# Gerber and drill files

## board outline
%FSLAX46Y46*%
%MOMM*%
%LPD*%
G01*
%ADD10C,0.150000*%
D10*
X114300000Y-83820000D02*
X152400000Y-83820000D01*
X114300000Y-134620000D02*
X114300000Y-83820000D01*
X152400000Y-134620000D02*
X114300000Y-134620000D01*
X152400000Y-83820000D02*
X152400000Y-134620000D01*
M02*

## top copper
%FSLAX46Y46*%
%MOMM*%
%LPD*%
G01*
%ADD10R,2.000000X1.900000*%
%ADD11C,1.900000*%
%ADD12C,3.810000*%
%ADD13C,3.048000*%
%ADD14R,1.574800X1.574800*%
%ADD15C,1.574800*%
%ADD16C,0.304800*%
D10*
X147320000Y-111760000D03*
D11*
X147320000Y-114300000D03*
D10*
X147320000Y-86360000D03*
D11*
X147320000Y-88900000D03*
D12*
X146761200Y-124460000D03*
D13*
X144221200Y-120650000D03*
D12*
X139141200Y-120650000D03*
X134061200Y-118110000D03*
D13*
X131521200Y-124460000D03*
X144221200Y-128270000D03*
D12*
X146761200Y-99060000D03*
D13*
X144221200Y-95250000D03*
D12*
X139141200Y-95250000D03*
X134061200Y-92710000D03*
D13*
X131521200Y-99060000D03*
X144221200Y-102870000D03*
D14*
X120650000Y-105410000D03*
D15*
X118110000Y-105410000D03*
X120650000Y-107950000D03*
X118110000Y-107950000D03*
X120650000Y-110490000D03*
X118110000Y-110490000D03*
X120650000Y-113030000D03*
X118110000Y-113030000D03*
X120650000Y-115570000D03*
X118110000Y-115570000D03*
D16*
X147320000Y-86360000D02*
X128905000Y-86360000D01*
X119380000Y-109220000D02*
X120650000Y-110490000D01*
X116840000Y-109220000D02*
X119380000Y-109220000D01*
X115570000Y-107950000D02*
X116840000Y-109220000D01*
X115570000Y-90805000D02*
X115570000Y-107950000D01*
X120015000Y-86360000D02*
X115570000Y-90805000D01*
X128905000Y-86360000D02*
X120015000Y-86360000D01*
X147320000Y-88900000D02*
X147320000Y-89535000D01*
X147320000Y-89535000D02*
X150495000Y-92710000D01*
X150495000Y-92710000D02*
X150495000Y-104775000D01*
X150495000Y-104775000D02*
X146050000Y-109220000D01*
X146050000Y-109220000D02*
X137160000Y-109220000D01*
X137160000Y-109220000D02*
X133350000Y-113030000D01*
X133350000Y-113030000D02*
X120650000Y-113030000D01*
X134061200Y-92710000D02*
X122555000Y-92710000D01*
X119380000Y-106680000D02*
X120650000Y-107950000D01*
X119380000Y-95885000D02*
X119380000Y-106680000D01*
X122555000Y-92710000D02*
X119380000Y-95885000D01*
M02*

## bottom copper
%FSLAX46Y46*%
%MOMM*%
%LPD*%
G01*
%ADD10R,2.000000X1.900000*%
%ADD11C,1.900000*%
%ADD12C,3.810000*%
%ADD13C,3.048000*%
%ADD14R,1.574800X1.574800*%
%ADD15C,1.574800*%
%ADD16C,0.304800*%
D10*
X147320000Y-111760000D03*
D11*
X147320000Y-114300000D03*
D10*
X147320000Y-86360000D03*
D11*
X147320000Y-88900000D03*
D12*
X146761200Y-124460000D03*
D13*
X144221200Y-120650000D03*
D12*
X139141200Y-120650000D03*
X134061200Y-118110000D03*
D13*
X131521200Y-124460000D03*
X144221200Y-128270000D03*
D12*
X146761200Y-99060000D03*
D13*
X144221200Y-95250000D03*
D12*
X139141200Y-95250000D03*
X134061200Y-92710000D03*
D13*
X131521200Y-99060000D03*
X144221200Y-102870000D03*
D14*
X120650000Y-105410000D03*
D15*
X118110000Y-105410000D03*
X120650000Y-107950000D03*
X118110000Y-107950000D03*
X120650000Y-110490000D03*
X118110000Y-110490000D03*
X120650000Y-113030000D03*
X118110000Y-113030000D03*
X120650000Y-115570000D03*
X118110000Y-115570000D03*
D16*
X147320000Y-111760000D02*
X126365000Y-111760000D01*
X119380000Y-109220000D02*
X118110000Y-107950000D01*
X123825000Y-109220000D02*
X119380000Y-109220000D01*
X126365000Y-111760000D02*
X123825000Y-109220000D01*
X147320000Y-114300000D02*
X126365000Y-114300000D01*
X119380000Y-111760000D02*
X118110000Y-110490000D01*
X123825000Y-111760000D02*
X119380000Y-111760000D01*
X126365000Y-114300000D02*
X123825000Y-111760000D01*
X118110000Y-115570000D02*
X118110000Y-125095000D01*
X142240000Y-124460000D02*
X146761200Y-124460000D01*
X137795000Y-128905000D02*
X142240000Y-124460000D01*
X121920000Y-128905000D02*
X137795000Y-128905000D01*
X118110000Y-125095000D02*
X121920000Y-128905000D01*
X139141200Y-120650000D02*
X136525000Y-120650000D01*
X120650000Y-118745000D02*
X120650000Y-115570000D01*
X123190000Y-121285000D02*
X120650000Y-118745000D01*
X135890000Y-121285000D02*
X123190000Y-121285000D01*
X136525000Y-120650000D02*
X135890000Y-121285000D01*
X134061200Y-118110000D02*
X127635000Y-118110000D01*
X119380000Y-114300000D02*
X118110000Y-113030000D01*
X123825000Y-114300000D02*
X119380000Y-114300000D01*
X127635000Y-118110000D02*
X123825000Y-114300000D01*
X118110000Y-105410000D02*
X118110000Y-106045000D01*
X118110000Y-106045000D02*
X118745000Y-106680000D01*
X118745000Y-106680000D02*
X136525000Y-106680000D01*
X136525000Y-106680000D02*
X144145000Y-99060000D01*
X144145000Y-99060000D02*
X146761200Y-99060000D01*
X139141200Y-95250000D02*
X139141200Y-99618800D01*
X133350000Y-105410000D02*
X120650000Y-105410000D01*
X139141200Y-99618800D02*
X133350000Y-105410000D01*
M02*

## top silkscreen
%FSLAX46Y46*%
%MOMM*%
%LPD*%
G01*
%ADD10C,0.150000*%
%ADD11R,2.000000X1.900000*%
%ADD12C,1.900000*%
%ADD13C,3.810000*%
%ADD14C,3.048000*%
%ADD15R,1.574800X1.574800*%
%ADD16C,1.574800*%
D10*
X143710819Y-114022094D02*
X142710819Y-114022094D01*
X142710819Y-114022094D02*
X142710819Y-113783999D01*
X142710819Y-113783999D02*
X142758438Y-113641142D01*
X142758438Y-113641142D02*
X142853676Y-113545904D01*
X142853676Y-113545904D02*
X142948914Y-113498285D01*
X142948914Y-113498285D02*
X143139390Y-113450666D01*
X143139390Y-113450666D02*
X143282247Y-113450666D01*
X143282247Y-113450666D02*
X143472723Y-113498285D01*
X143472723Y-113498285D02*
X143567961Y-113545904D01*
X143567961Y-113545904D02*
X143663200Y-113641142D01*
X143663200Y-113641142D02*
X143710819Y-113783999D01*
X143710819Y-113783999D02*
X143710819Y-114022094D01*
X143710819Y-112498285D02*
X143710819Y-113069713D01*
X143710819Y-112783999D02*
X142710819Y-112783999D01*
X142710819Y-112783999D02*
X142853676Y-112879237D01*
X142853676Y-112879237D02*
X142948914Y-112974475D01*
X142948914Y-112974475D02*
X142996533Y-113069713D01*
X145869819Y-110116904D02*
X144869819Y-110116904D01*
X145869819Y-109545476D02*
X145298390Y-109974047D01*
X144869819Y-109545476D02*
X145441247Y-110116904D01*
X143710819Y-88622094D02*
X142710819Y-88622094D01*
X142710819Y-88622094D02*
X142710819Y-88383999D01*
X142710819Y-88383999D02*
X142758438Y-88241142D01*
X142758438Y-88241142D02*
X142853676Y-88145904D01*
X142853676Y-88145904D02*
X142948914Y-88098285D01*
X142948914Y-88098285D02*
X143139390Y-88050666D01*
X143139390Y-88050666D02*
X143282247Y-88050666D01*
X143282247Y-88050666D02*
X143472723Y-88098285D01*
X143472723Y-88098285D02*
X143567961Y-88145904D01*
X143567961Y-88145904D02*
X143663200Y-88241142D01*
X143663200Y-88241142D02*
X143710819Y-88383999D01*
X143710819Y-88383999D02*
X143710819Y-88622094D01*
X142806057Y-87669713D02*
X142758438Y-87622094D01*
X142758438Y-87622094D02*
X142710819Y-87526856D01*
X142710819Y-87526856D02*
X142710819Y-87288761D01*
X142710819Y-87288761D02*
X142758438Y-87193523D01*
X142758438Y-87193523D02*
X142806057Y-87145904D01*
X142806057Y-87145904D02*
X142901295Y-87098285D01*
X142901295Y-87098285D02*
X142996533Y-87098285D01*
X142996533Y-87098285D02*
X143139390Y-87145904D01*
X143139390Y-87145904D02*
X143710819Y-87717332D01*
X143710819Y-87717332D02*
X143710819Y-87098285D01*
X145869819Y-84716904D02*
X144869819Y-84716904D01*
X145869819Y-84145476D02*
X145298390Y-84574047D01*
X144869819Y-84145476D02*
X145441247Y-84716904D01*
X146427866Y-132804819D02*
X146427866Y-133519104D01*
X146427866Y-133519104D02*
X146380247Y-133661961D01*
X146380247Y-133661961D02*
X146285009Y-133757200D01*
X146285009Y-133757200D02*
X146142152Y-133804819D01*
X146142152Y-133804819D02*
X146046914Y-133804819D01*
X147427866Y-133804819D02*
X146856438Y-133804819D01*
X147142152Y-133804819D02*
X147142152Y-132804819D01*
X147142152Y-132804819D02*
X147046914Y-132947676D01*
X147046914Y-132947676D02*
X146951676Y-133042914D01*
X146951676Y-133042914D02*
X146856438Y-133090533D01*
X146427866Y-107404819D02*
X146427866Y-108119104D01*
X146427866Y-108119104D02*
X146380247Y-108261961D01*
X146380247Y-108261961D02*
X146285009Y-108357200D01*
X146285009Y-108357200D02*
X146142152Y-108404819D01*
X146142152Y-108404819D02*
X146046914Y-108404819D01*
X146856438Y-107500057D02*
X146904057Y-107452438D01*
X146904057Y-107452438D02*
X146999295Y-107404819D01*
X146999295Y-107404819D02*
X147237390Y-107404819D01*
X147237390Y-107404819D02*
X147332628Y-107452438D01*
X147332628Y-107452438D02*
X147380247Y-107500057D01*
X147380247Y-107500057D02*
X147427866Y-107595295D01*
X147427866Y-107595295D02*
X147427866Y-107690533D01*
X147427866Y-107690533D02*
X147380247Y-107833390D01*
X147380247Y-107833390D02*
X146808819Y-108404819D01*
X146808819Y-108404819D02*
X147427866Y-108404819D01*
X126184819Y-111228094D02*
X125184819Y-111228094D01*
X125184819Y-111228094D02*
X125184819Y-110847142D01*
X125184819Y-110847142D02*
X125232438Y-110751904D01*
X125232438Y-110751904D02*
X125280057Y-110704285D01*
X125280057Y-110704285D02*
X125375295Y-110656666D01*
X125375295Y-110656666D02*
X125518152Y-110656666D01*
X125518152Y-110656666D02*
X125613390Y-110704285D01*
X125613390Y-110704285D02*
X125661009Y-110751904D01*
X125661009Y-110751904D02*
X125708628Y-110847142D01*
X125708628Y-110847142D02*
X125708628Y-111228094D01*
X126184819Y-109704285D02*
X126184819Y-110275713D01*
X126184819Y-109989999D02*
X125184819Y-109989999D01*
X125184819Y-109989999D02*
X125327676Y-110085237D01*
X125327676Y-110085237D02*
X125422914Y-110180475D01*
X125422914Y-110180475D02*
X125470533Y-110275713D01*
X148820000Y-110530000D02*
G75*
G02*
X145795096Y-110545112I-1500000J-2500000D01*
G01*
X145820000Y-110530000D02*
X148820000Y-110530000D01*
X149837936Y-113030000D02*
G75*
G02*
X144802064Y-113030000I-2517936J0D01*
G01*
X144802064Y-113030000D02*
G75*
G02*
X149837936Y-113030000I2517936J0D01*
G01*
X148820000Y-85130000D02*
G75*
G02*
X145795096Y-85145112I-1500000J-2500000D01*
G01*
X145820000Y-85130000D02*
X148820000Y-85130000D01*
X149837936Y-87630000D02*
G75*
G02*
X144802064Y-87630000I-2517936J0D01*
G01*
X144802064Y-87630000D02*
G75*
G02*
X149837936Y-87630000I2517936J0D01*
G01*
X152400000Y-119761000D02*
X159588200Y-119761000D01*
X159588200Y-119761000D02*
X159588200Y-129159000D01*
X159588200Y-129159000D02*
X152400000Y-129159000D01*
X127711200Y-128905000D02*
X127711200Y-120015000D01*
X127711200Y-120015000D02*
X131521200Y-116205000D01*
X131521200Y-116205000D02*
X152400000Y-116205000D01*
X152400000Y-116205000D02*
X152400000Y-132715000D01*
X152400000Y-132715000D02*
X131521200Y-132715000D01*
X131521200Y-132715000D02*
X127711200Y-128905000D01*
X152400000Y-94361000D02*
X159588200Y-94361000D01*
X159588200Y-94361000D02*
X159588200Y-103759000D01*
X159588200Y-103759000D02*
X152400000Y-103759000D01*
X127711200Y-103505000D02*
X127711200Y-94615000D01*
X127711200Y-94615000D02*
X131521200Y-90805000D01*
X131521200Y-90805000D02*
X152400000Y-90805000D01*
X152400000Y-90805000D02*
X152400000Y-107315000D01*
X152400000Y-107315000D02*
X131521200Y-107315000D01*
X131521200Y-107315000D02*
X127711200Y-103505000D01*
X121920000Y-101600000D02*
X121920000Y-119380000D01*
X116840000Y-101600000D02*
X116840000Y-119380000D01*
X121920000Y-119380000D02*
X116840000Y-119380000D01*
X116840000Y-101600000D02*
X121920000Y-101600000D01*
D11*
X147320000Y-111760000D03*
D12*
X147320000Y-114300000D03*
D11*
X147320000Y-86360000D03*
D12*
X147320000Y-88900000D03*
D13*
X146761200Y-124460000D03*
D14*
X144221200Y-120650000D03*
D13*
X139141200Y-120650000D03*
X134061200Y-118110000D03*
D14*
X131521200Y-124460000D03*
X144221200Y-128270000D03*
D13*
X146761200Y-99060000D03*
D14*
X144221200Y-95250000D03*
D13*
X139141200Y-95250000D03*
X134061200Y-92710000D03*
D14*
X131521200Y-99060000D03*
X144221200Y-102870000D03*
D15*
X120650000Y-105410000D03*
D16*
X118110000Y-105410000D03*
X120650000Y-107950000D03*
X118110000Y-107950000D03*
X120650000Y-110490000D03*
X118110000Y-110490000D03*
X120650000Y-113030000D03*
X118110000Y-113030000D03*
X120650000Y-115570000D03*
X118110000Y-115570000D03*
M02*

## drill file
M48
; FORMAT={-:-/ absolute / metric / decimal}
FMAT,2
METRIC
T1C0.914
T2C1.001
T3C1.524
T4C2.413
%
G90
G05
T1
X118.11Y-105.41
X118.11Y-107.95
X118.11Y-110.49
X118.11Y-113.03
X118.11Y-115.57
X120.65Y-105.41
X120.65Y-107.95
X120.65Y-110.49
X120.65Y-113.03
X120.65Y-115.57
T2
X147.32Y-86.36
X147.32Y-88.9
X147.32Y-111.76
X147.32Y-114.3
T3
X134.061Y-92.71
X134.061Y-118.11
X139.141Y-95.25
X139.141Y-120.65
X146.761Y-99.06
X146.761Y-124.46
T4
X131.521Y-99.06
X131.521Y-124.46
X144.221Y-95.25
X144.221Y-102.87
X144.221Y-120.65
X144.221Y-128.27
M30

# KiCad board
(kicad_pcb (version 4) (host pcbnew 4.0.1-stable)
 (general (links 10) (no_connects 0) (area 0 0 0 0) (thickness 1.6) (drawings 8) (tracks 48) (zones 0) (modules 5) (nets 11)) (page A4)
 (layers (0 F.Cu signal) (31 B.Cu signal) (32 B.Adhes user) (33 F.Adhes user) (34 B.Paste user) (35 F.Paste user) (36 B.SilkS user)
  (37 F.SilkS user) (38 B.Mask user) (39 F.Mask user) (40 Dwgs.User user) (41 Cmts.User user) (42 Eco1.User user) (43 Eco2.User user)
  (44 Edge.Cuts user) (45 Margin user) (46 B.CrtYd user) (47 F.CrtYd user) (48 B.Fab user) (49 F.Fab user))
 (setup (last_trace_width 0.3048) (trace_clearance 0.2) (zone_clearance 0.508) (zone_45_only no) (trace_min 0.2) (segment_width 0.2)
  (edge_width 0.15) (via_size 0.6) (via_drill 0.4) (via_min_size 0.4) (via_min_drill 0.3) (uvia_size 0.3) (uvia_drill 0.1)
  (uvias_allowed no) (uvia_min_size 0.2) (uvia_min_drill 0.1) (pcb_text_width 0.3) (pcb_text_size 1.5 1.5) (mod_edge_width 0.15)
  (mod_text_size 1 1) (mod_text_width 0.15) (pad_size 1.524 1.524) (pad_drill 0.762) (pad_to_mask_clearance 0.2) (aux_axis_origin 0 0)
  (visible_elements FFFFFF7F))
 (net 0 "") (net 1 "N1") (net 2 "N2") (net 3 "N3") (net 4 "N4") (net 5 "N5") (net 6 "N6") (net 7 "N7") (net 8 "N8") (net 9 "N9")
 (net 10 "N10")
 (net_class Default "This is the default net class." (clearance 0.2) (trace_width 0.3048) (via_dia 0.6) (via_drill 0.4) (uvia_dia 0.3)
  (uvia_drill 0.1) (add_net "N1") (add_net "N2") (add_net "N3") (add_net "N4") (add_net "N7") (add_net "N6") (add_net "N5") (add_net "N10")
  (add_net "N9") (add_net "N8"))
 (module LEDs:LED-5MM (layer F.Cu) (at 147.32 111.76 270)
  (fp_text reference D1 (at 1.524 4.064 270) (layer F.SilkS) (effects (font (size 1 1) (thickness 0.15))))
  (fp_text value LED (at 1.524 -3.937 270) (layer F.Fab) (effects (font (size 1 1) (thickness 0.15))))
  (fp_arc (start 1.27 0) (end -1.23 -1.5) (angle 297.5) (layer F.SilkS) (width 0.15))
  (fp_line (start -1.23 1.5) (end -1.23 -1.5) (layer F.SilkS) (width 0.15))
  (fp_circle (center 1.27 0) (end 0.97 -2.5) (layer F.SilkS) (width 0.15))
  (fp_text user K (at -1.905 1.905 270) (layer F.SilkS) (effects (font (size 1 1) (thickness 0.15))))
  (pad 1 thru_hole rect (at 0 0) (size 2 1.9) (drill 1.00076) (layers *.Cu *.Mask F.SilkS) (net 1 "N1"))
  (pad 2 thru_hole circle (at 2.54 0 270) (size 1.9 1.9) (drill 1.00076) (layers *.Cu *.Mask F.SilkS) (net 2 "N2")))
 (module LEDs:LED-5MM (layer F.Cu) (at 147.32 86.36 270)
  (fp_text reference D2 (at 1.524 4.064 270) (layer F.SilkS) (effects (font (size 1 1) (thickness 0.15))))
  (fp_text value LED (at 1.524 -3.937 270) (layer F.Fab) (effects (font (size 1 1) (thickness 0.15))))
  (fp_arc (start 1.27 0) (end -1.23 -1.5) (angle 297.5) (layer F.SilkS) (width 0.15))
  (fp_line (start -1.23 1.5) (end -1.23 -1.5) (layer F.SilkS) (width 0.15))
  (fp_circle (center 1.27 0) (end 0.97 -2.5) (layer F.SilkS) (width 0.15))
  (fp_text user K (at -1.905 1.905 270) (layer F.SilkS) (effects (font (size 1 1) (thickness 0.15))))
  (pad 1 thru_hole rect (at 0 0) (size 2 1.9) (drill 1.00076) (layers *.Cu *.Mask F.SilkS) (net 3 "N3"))
  (pad 2 thru_hole circle (at 2.54 0 270) (size 1.9 1.9) (drill 1.00076) (layers *.Cu *.Mask F.SilkS) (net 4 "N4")))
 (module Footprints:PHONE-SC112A (layer F.Cu) (at 152.4 124.46)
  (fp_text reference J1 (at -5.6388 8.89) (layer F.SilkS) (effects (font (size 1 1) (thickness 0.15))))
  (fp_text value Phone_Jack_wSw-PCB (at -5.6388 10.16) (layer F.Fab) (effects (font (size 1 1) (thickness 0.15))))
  (fp_line (start 0 -4.699) (end 7.1882 -4.699) (layer F.SilkS) (width 0.15))
  (fp_line (start 7.1882 -4.699) (end 7.1882 4.699) (layer F.SilkS) (width 0.15))
  (fp_line (start 7.1882 4.699) (end 0 4.699) (layer F.SilkS) (width 0.15))
  (fp_line (start -24.6888 4.445) (end -24.6888 -4.445) (layer F.SilkS) (width 0.15))
  (fp_line (start -24.6888 -4.445) (end -20.8788 -8.255) (layer F.SilkS) (width 0.15))
  (fp_line (start -20.8788 -8.255) (end 0 -8.255) (layer F.SilkS) (width 0.15))
  (fp_line (start 0 -8.255) (end 0 8.255) (layer F.SilkS) (width 0.15))
  (fp_line (start 0 8.255) (end -20.8788 8.255) (layer F.SilkS) (width 0.15))
  (fp_line (start -20.8788 8.255) (end -24.6888 4.445) (layer F.SilkS) (width 0.15))
  (pad 3 thru_hole circle (at -5.6388 0) (size 3.81 3.81) (drill 1.524) (layers *.Cu *.Mask F.SilkS) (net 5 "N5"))
  (pad "" thru_hole circle (at -8.1788 -3.81) (size 3.048 3.048) (drill 2.413) (layers *.Cu *.Mask F.SilkS))
  (pad 2 thru_hole circle (at -13.2588 -3.81) (size 3.81 3.81) (drill 1.524) (layers *.Cu *.Mask F.SilkS) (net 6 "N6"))
  (pad 1 thru_hole circle (at -18.3388 -6.35) (size 3.81 3.81) (drill 1.524) (layers *.Cu *.Mask F.SilkS) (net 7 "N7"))
  (pad "" thru_hole circle (at -20.8788 0) (size 3.048 3.048) (drill 2.413) (layers *.Cu *.Mask F.SilkS))
  (pad "" thru_hole circle (at -8.1788 3.81) (size 3.048 3.048) (drill 2.413) (layers *.Cu *.Mask F.SilkS)))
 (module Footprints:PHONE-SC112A (layer F.Cu) (at 152.4 99.06)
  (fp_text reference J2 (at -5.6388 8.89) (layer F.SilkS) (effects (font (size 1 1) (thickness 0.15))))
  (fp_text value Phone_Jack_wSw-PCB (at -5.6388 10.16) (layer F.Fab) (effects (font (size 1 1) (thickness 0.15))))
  (fp_line (start 0 -4.699) (end 7.1882 -4.699) (layer F.SilkS) (width 0.15))
  (fp_line (start 7.1882 -4.699) (end 7.1882 4.699) (layer F.SilkS) (width 0.15))
  (fp_line (start 7.1882 4.699) (end 0 4.699) (layer F.SilkS) (width 0.15))
  (fp_line (start -24.6888 4.445) (end -24.6888 -4.445) (layer F.SilkS) (width 0.15))
  (fp_line (start -24.6888 -4.445) (end -20.8788 -8.255) (layer F.SilkS) (width 0.15))
  (fp_line (start -20.8788 -8.255) (end 0 -8.255) (layer F.SilkS) (width 0.15))
  (fp_line (start 0 -8.255) (end 0 8.255) (layer F.SilkS) (width 0.15))
  (fp_line (start 0 8.255) (end -20.8788 8.255) (layer F.SilkS) (width 0.15))
  (fp_line (start -20.8788 8.255) (end -24.6888 4.445) (layer F.SilkS) (width 0.15))
  (pad 3 thru_hole circle (at -5.6388 0) (size 3.81 3.81) (drill 1.524) (layers *.Cu *.Mask F.SilkS) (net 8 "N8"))
  (pad "" thru_hole circle (at -8.1788 -3.81) (size 3.048 3.048) (drill 2.413) (layers *.Cu *.Mask F.SilkS))
  (pad 2 thru_hole circle (at -13.2588 -3.81) (size 3.81 3.81) (drill 1.524) (layers *.Cu *.Mask F.SilkS) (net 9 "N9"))
  (pad 1 thru_hole circle (at -18.3388 -6.35) (size 3.81 3.81) (drill 1.524) (layers *.Cu *.Mask F.SilkS) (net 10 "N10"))
  (pad "" thru_hole circle (at -20.8788 0) (size 3.048 3.048) (drill 2.413) (layers *.Cu *.Mask F.SilkS))
  (pad "" thru_hole circle (at -8.1788 3.81) (size 3.048 3.048) (drill 2.413) (layers *.Cu *.Mask F.SilkS)))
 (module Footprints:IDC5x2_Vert (layer F.Cu) (at 119.38 114.3 90)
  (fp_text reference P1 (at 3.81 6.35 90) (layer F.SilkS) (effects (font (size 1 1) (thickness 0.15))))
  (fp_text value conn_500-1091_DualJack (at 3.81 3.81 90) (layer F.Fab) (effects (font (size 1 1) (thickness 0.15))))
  (fp_line (start 12.7 2.54) (end -5.08 2.54) (layer F.SilkS) (width 0.15))
  (fp_line (start 12.7 -2.54) (end -5.08 -2.54) (layer F.SilkS) (width 0.15))
  (fp_line (start -5.08 2.54) (end -5.08 -2.54) (layer F.SilkS) (width 0.15))
  (fp_line (start 12.7 -2.54) (end 12.7 2.54) (layer F.SilkS) (width 0.15))
  (pad 1 thru_hole rect (at 8.89 1.27 90) (size 1.5748 1.5748) (drill 0.9144) (layers *.Cu *.Mask F.SilkS) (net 9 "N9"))
  (pad 2 thru_hole circle (at 8.89 -1.27 90) (size 1.5748 1.5748) (drill 0.9144) (layers *.Cu *.Mask F.SilkS) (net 8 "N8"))
  (pad 3 thru_hole circle (at 6.35 1.27 90) (size 1.5748 1.5748) (drill 0.9144) (layers *.Cu *.Mask F.SilkS) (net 10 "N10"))
  (pad 4 thru_hole circle (at 6.35 -1.27 90) (size 1.5748 1.5748) (drill 0.9144) (layers *.Cu *.Mask F.SilkS) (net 1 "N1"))
  (pad 5 thru_hole circle (at 3.81 1.27 90) (size 1.5748 1.5748) (drill 0.9144) (layers *.Cu *.Mask F.SilkS) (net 3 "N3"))
  (pad 6 thru_hole circle (at 3.81 -1.27 90) (size 1.5748 1.5748) (drill 0.9144) (layers *.Cu *.Mask F.SilkS) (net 2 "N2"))
  (pad 7 thru_hole circle (at 1.27 1.27 90) (size 1.5748 1.5748) (drill 0.9144) (layers *.Cu *.Mask F.SilkS) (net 4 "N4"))
  (pad 8 thru_hole circle (at 1.27 -1.27 90) (size 1.5748 1.5748) (drill 0.9144) (layers *.Cu *.Mask F.SilkS) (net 7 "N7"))
  (pad 9 thru_hole circle (at -1.27 1.27 90) (size 1.5748 1.5748) (drill 0.9144) (layers *.Cu *.Mask F.SilkS) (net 6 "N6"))
  (pad 10 thru_hole circle (at -1.27 -1.27 90) (size 1.5748 1.5748) (drill 0.9144) (layers *.Cu *.Mask F.SilkS) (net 5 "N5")))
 (gr_line (start 114.3 83.82) (end 152.4 83.82) (angle 90) (layer Edge.Cuts) (width 0.15))
 (gr_line (start 114.3 134.62) (end 114.3 83.82) (angle 90) (layer Edge.Cuts) (width 0.15))
 (gr_line (start 152.4 134.62) (end 114.3 134.62) (angle 90) (layer Edge.Cuts) (width 0.15))
 (gr_line (start 152.4 83.82) (end 152.4 134.62) (angle 90) (layer Edge.Cuts) (width 0.15))
 (segment (start 147.32 111.76) (end 126.365 111.76) (width 0.3048) (layer B.Cu) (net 1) (status 400000))
 (segment (start 119.38 109.22) (end 118.11 107.95) (width 0.3048) (layer B.Cu) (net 1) (status 800000))
 (segment (start 123.825 109.22) (end 119.38 109.22) (width 0.3048) (layer B.Cu) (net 1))
 (segment (start 126.365 111.76) (end 123.825 109.22) (width 0.3048) (layer B.Cu) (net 1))
 (segment (start 147.32 114.3) (end 126.365 114.3) (width 0.3048) (layer B.Cu) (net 2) (status 400000))
 (segment (start 119.38 111.76) (end 118.11 110.49) (width 0.3048) (layer B.Cu) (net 2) (status 800000))
 (segment (start 123.825 111.76) (end 119.38 111.76) (width 0.3048) (layer B.Cu) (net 2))
 (segment (start 126.365 114.3) (end 123.825 111.76) (width 0.3048) (layer B.Cu) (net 2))
 (segment (start 147.32 86.36) (end 128.905 86.36) (width 0.3048) (layer F.Cu) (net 3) (status 400000))
 (segment (start 119.38 109.22) (end 120.65 110.49) (width 0.3048) (layer F.Cu) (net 3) (status 800000))
 (segment (start 116.84 109.22) (end 119.38 109.22) (width 0.3048) (layer F.Cu) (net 3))
 (segment (start 115.57 107.95) (end 116.84 109.22) (width 0.3048) (layer F.Cu) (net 3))
 (segment (start 115.57 90.805) (end 115.57 107.95) (width 0.3048) (layer F.Cu) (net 3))
 (segment (start 120.015 86.36) (end 115.57 90.805) (width 0.3048) (layer F.Cu) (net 3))
 (segment (start 128.905 86.36) (end 120.015 86.36) (width 0.3048) (layer F.Cu) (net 3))
 (segment (start 147.32 88.9) (end 147.32 89.535) (width 0.3048) (layer F.Cu) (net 4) (status C00000))
 (segment (start 147.32 89.535) (end 150.495 92.71) (width 0.3048) (layer F.Cu) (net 4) (status 400000))
 (segment (start 150.495 92.71) (end 150.495 104.775) (width 0.3048) (layer F.Cu) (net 4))
 (segment (start 150.495 104.775) (end 146.05 109.22) (width 0.3048) (layer F.Cu) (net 4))
 (segment (start 146.05 109.22) (end 137.16 109.22) (width 0.3048) (layer F.Cu) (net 4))
 (segment (start 137.16 109.22) (end 133.35 113.03) (width 0.3048) (layer F.Cu) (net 4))
 (segment (start 133.35 113.03) (end 120.65 113.03) (width 0.3048) (layer F.Cu) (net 4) (status 800000))
 (segment (start 118.11 115.57) (end 118.11 125.095) (width 0.3048) (layer B.Cu) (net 5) (status 400000))
 (segment (start 142.24 124.46) (end 146.7612 124.46) (width 0.3048) (layer B.Cu) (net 5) (status 800000))
 (segment (start 137.795 128.905) (end 142.24 124.46) (width 0.3048) (layer B.Cu) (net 5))
 (segment (start 121.92 128.905) (end 137.795 128.905) (width 0.3048) (layer B.Cu) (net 5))
 (segment (start 118.11 125.095) (end 121.92 128.905) (width 0.3048) (layer B.Cu) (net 5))
 (segment (start 139.1412 120.65) (end 136.525 120.65) (width 0.3048) (layer B.Cu) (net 6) (status 400000))
 (segment (start 120.65 118.745) (end 120.65 115.57) (width 0.3048) (layer B.Cu) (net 6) (status 800000))
 (segment (start 123.19 121.285) (end 120.65 118.745) (width 0.3048) (layer B.Cu) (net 6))
 (segment (start 135.89 121.285) (end 123.19 121.285) (width 0.3048) (layer B.Cu) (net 6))
 (segment (start 136.525 120.65) (end 135.89 121.285) (width 0.3048) (layer B.Cu) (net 6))
 (segment (start 134.0612 118.11) (end 127.635 118.11) (width 0.3048) (layer B.Cu) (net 7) (status 400000))
 (segment (start 119.38 114.3) (end 118.11 113.03) (width 0.3048) (layer B.Cu) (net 7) (status 800000))
 (segment (start 123.825 114.3) (end 119.38 114.3) (width 0.3048) (layer B.Cu) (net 7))
 (segment (start 127.635 118.11) (end 123.825 114.3) (width 0.3048) (layer B.Cu) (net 7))
 (segment (start 118.11 105.41) (end 118.11 106.045) (width 0.3048) (layer B.Cu) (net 8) (status C00000))
 (segment (start 118.11 106.045) (end 118.745 106.68) (width 0.3048) (layer B.Cu) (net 8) (status 400000))
 (segment (start 118.745 106.68) (end 136.525 106.68) (width 0.3048) (layer B.Cu) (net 8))
 (segment (start 136.525 106.68) (end 144.145 99.06) (width 0.3048) (layer B.Cu) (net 8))
 (segment (start 144.145 99.06) (end 146.7612 99.06) (width 0.3048) (layer B.Cu) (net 8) (status 800000))
 (segment (start 139.1412 95.25) (end 139.1412 99.6188) (width 0.3048) (layer B.Cu) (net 9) (status 400000))
 (segment (start 133.35 105.41) (end 120.65 105.41) (width 0.3048) (layer B.Cu) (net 9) (status 800000))
 (segment (start 139.1412 99.6188) (end 133.35 105.41) (width 0.3048) (layer B.Cu) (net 9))
 (segment (start 134.0612 92.71) (end 122.555 92.71) (width 0.3048) (layer F.Cu) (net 10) (status 400000))
 (segment (start 119.38 106.68) (end 120.65 107.95) (width 0.3048) (layer F.Cu) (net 10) (status 800000))
 (segment (start 119.38 95.885) (end 119.38 106.68) (width 0.3048) (layer F.Cu) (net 10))
 (segment (start 122.555 92.71) (end 119.38 95.885) (width 0.3048) (layer F.Cu) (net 10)))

